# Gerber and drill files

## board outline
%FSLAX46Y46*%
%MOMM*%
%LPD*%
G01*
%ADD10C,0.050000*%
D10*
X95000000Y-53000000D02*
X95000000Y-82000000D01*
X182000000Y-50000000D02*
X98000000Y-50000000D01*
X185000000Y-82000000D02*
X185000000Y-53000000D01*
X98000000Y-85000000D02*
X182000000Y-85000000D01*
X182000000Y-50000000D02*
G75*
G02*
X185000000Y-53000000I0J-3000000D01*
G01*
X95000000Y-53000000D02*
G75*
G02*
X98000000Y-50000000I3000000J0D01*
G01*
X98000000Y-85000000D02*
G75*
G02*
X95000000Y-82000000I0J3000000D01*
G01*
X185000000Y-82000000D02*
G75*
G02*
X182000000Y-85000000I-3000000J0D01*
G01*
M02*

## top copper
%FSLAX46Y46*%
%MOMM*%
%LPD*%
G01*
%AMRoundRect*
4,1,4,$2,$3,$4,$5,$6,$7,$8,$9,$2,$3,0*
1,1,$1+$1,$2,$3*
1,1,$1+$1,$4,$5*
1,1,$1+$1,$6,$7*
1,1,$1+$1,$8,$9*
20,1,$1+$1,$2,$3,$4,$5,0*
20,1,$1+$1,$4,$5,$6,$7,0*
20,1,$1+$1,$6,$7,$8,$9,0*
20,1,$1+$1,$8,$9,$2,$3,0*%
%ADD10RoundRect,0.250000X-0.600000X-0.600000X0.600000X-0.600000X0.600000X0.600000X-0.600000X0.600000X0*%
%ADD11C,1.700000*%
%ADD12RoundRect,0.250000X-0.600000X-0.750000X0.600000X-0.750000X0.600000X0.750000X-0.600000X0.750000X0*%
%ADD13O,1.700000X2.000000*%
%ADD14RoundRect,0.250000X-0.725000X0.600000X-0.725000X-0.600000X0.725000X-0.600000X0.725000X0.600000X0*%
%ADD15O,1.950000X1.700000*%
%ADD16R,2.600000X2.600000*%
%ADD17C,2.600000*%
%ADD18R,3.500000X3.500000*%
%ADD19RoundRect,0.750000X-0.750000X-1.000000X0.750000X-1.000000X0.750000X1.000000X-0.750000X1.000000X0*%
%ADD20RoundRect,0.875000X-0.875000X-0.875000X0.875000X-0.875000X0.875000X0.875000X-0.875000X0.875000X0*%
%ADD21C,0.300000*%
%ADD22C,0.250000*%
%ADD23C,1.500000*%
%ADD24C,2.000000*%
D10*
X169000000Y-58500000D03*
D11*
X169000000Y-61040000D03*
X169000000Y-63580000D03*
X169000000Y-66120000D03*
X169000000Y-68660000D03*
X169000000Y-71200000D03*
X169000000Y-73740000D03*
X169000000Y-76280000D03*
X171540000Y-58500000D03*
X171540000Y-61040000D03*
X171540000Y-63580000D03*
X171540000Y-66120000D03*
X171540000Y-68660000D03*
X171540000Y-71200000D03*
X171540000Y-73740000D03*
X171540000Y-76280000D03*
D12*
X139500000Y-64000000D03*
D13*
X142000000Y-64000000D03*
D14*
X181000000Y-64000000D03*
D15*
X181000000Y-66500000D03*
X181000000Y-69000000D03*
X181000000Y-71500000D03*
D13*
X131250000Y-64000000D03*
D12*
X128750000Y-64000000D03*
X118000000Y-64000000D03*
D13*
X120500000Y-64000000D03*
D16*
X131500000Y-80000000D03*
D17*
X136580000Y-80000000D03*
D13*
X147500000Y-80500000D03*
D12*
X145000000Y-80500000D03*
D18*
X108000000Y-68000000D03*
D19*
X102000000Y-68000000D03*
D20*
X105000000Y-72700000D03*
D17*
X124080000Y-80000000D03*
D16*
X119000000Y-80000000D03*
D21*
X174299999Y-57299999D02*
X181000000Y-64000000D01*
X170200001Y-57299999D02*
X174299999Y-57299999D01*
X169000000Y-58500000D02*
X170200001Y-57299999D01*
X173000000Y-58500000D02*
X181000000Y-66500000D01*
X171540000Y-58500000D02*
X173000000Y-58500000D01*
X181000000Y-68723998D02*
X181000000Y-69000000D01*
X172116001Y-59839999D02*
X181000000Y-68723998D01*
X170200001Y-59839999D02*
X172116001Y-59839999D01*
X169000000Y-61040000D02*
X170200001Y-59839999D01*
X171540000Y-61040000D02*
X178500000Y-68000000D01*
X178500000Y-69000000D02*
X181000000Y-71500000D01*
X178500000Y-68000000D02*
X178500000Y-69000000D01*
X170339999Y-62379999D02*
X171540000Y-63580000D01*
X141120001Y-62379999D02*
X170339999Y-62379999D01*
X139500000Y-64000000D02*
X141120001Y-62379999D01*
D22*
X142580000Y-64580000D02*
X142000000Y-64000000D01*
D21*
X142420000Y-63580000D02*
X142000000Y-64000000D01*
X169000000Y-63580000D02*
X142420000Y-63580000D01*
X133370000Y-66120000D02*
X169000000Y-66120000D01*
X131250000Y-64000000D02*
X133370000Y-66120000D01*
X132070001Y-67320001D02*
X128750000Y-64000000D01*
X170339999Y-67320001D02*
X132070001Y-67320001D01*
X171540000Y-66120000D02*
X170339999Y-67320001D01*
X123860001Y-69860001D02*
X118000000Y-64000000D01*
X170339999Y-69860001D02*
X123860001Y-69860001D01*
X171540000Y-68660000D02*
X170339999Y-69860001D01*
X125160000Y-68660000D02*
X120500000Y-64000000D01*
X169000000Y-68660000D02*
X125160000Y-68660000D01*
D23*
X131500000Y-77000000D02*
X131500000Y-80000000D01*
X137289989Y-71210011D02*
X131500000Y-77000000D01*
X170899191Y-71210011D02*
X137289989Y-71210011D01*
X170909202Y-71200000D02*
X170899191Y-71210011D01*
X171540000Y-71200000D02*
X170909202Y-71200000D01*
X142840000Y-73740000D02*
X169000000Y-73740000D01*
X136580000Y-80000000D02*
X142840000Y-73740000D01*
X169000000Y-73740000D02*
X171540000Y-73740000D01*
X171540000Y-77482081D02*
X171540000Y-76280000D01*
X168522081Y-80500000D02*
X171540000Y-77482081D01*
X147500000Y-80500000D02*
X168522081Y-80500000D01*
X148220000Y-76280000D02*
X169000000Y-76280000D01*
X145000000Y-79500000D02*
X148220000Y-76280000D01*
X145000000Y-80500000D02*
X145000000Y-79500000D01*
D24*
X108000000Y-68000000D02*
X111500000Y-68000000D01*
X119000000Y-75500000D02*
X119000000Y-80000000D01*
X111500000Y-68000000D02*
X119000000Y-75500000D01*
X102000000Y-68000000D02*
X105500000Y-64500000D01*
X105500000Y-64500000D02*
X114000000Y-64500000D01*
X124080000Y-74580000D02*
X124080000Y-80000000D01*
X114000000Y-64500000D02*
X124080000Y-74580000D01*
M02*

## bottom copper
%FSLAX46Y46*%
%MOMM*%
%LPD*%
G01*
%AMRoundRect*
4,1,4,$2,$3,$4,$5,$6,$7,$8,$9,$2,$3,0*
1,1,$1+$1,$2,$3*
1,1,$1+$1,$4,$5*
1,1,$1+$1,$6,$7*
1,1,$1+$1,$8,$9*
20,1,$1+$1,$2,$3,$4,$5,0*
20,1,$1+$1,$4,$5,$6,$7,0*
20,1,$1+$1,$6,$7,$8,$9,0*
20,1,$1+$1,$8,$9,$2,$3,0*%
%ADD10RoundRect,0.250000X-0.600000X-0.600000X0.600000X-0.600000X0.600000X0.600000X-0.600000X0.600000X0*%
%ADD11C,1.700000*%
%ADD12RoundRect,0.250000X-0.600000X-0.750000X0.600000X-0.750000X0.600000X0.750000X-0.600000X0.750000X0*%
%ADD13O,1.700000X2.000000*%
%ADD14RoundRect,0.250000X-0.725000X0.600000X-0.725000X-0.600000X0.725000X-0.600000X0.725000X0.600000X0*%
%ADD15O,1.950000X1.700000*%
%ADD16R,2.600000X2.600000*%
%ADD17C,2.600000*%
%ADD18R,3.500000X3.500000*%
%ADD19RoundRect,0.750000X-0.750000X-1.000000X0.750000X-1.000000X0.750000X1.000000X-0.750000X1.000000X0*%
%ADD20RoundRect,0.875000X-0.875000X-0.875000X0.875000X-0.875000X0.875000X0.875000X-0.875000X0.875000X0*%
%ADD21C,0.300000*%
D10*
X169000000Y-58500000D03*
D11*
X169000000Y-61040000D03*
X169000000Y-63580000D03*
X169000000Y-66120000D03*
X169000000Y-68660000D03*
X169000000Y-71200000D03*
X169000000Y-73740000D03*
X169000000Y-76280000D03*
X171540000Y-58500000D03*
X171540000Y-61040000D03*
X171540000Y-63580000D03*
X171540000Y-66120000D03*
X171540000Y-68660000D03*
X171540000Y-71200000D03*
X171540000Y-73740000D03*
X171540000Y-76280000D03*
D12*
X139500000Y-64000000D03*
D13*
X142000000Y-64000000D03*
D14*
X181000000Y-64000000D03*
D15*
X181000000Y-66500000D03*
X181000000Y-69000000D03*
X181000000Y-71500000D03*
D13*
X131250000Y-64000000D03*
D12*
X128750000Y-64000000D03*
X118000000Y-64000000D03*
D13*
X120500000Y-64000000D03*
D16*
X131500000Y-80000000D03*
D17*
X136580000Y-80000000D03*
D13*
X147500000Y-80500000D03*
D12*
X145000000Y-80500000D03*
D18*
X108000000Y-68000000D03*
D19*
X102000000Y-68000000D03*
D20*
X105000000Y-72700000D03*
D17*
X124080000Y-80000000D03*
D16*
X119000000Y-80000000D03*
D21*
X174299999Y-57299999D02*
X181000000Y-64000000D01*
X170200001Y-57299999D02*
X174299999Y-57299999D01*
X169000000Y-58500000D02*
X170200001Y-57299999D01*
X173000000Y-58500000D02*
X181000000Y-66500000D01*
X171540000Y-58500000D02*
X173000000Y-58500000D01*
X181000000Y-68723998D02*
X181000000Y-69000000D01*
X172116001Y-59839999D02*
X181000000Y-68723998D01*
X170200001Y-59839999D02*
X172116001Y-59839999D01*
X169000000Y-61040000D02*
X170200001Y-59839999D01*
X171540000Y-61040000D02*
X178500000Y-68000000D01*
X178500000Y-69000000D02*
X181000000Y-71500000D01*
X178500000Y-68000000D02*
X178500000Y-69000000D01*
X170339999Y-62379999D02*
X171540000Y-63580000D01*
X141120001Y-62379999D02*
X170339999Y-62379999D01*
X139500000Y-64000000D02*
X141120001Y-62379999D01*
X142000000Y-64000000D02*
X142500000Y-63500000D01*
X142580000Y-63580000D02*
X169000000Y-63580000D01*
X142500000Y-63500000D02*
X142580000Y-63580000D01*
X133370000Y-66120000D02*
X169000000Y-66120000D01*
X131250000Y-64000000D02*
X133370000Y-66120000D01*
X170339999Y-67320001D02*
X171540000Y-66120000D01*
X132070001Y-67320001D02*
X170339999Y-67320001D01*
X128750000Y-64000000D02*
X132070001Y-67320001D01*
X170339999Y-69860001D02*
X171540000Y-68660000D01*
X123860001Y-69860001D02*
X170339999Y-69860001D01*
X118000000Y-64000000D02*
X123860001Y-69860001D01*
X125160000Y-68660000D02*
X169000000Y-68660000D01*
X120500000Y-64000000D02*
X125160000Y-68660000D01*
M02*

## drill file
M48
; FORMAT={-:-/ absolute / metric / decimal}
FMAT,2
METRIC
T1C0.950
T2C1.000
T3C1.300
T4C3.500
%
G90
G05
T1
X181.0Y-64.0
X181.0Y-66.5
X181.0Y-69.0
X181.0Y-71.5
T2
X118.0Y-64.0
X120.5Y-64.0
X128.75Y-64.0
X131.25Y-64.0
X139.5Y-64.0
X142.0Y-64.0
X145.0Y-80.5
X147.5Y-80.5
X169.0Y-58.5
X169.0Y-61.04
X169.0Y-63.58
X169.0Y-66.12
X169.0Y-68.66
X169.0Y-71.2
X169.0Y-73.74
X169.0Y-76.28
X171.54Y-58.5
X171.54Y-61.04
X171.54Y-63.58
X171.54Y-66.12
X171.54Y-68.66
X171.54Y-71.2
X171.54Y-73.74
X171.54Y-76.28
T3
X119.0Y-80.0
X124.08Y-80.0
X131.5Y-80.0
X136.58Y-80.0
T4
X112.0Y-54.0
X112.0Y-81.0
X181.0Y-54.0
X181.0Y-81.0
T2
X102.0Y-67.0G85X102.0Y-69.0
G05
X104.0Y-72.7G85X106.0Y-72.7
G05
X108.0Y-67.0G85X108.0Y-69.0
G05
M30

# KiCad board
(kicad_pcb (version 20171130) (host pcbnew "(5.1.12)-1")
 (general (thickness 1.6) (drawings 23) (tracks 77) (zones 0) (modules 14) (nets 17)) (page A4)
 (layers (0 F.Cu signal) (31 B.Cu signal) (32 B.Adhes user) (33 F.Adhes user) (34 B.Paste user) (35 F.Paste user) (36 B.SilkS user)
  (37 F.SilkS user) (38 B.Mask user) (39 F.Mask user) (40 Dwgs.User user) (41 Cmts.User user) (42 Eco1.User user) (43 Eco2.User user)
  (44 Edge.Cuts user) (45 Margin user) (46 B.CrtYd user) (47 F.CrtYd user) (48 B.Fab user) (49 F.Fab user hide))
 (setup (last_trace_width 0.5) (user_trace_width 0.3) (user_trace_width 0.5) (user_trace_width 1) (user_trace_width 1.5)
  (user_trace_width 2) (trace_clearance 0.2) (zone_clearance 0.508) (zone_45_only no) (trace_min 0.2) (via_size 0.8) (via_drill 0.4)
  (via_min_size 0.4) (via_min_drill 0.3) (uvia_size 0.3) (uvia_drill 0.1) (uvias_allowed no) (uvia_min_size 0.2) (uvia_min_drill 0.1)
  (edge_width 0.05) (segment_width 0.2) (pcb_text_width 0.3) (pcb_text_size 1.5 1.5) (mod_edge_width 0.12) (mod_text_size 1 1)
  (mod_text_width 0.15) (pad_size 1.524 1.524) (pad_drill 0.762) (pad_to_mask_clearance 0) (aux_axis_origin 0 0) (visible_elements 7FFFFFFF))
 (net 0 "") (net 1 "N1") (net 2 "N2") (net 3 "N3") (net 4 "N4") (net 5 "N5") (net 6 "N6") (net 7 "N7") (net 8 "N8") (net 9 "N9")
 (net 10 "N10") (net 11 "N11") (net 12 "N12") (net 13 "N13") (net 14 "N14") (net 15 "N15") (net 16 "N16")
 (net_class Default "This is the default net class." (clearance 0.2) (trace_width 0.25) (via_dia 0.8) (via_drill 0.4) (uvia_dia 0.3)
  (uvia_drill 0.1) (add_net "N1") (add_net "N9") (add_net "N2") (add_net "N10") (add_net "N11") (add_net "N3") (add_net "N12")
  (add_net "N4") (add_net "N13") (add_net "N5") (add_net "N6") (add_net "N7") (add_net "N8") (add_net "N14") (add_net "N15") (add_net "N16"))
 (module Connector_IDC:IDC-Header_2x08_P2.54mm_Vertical (layer F.Cu) (at 169 58.5)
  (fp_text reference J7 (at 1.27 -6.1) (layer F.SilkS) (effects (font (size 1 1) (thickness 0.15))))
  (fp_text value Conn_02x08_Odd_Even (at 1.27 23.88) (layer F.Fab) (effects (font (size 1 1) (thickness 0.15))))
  (pad 1 thru_hole roundrect (at 0 0) (size 1.7 1.7) (drill 1) (layers *.Cu *.Mask) (roundrect_rratio 0.1470588235294118) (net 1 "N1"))
  (pad 3 thru_hole circle (at 0 2.54) (size 1.7 1.7) (drill 1) (layers *.Cu *.Mask) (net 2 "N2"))
  (pad 5 thru_hole circle (at 0 5.08) (size 1.7 1.7) (drill 1) (layers *.Cu *.Mask) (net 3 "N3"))
  (pad 7 thru_hole circle (at 0 7.62) (size 1.7 1.7) (drill 1) (layers *.Cu *.Mask) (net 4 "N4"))
  (pad 9 thru_hole circle (at 0 10.16) (size 1.7 1.7) (drill 1) (layers *.Cu *.Mask) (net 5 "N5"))
  (pad 11 thru_hole circle (at 0 12.7) (size 1.7 1.7) (drill 1) (layers *.Cu *.Mask) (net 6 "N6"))
  (pad 13 thru_hole circle (at 0 15.24) (size 1.7 1.7) (drill 1) (layers *.Cu *.Mask) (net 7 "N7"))
  (pad 15 thru_hole circle (at 0 17.78) (size 1.7 1.7) (drill 1) (layers *.Cu *.Mask) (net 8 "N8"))
  (pad 2 thru_hole circle (at 2.54 0) (size 1.7 1.7) (drill 1) (layers *.Cu *.Mask) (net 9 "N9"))
  (pad 4 thru_hole circle (at 2.54 2.54) (size 1.7 1.7) (drill 1) (layers *.Cu *.Mask) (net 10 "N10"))
  (pad 6 thru_hole circle (at 2.54 5.08) (size 1.7 1.7) (drill 1) (layers *.Cu *.Mask) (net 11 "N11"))
  (pad 8 thru_hole circle (at 2.54 7.62) (size 1.7 1.7) (drill 1) (layers *.Cu *.Mask) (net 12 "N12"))
  (pad 10 thru_hole circle (at 2.54 10.16) (size 1.7 1.7) (drill 1) (layers *.Cu *.Mask) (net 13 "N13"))
  (pad 12 thru_hole circle (at 2.54 12.7) (size 1.7 1.7) (drill 1) (layers *.Cu *.Mask) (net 6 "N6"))
  (pad 14 thru_hole circle (at 2.54 15.24) (size 1.7 1.7) (drill 1) (layers *.Cu *.Mask) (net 7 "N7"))
  (pad 16 thru_hole circle (at 2.54 17.78) (size 1.7 1.7) (drill 1) (layers *.Cu *.Mask) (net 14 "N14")))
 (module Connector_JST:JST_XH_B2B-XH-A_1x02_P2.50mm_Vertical (layer F.Cu) (at 139.5 64)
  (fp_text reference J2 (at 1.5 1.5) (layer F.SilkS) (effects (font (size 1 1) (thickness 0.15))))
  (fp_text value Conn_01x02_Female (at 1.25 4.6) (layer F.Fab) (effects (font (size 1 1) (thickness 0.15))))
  (pad 1 thru_hole roundrect (at 0 0) (size 1.7 2) (drill 1) (layers *.Cu *.Mask) (roundrect_rratio 0.1470588235294118) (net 11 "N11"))
  (pad 2 thru_hole oval (at 2.5 0) (size 1.7 2) (drill 1) (layers *.Cu *.Mask) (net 3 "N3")))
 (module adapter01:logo (layer F.Cu) (at 155.5 67.5)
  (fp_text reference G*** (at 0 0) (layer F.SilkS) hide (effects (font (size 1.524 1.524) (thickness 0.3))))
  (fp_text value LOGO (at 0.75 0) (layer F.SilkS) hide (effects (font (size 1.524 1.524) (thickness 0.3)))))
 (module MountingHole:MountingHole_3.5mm (layer F.Cu) (at 181 54)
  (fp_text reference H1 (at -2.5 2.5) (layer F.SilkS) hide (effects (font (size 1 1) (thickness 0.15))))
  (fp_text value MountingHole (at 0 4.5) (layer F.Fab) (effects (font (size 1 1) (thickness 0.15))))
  (pad 1 np_thru_hole circle (at 0 0) (size 3.5 3.5) (drill 3.5) (layers *.Cu *.Mask)))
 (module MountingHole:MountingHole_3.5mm (layer F.Cu) (at 112 81)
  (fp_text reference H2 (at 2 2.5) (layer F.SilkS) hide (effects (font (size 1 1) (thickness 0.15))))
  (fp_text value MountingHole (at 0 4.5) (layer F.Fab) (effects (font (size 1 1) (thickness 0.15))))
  (pad 1 np_thru_hole circle (at 0 0) (size 3.5 3.5) (drill 3.5) (layers *.Cu *.Mask)))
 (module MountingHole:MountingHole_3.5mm (layer F.Cu) (at 181 81)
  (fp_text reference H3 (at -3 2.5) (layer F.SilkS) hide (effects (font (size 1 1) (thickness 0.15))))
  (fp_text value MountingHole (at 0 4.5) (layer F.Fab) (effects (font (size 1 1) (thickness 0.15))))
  (pad 1 np_thru_hole circle (at 0 0) (size 3.5 3.5) (drill 3.5) (layers *.Cu *.Mask)))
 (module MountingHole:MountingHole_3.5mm (layer F.Cu) (at 112 54)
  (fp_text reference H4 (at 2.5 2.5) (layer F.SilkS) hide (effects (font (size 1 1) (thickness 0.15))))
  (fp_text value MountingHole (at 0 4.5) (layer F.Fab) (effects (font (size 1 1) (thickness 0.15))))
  (pad 1 np_thru_hole circle (at 0 0) (size 3.5 3.5) (drill 3.5) (layers *.Cu *.Mask)))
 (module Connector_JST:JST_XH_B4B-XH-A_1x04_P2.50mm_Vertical (layer F.Cu) (at 181 64 270)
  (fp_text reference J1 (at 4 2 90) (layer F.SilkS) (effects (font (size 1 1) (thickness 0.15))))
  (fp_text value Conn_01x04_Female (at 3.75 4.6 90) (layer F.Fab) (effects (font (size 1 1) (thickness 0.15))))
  (pad 1 thru_hole roundrect (at 0 0 270) (size 1.7 1.95) (drill 0.95) (layers *.Cu *.Mask) (roundrect_rratio 0.1470588235294118)
   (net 1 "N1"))
  (pad 2 thru_hole oval (at 2.5 0 270) (size 1.7 1.95) (drill 0.95) (layers *.Cu *.Mask) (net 9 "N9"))
  (pad 3 thru_hole oval (at 5 0 270) (size 1.7 1.95) (drill 0.95) (layers *.Cu *.Mask) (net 2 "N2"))
  (pad 4 thru_hole oval (at 7.5 0 270) (size 1.7 1.95) (drill 0.95) (layers *.Cu *.Mask) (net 10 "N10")))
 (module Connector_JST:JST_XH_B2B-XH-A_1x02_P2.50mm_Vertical (layer F.Cu) (at 128.75 64)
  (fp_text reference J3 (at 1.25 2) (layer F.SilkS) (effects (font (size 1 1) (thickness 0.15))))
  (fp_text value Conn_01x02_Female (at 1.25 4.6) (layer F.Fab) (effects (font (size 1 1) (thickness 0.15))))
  (pad 2 thru_hole oval (at 2.5 0) (size 1.7 2) (drill 1) (layers *.Cu *.Mask) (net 4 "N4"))
  (pad 1 thru_hole roundrect (at 0 0) (size 1.7 2) (drill 1) (layers *.Cu *.Mask) (roundrect_rratio 0.1470588235294118) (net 12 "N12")))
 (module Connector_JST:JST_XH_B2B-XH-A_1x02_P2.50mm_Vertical (layer F.Cu) (at 118 64)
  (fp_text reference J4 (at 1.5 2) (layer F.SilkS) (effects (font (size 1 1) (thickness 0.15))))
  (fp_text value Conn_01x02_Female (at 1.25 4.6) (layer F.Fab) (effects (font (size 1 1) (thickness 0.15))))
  (pad 1 thru_hole roundrect (at 0 0) (size 1.7 2) (drill 1) (layers *.Cu *.Mask) (roundrect_rratio 0.1470588235294118) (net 13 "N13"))
  (pad 2 thru_hole oval (at 2.5 0) (size 1.7 2) (drill 1) (layers *.Cu *.Mask) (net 5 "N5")))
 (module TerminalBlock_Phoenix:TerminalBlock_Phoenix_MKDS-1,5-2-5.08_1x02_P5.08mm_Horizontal (layer F.Cu) (at 131.5 80)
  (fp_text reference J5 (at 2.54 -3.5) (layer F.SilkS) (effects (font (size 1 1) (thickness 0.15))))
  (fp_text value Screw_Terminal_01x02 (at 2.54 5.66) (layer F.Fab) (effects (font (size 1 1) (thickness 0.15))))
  (pad 1 thru_hole rect (at 0 0) (size 2.6 2.6) (drill 1.3) (layers *.Cu *.Mask) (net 6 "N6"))
  (pad 2 thru_hole circle (at 5.08 0) (size 2.6 2.6) (drill 1.3) (layers *.Cu *.Mask) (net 7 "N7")))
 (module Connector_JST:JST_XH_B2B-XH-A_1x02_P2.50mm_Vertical (layer F.Cu) (at 145 80.5)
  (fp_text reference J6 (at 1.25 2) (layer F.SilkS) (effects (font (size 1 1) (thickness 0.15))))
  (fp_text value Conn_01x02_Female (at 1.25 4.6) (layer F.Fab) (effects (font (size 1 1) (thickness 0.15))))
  (pad 2 thru_hole oval (at 2.5 0) (size 1.7 2) (drill 1) (layers *.Cu *.Mask) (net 14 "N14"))
  (pad 1 thru_hole roundrect (at 0 0) (size 1.7 2) (drill 1) (layers *.Cu *.Mask) (roundrect_rratio 0.1470588235294118) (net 8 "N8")))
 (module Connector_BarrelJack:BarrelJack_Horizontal (layer F.Cu) (at 108 68)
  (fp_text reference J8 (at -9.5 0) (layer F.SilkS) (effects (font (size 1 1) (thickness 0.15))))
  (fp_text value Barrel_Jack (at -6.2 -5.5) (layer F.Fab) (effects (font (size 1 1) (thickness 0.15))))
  (pad 1 thru_hole rect (at 0 0) (size 3.5 3.5) (drill oval 1 3) (layers *.Cu *.Mask) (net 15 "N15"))
  (pad 2 thru_hole roundrect (at -6 0) (size 3 3.5) (drill oval 1 3) (layers *.Cu *.Mask) (roundrect_rratio 0.25) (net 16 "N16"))
  (pad 3 thru_hole roundrect (at -3 4.7) (size 3.5 3.5) (drill oval 3 1) (layers *.Cu *.Mask) (roundrect_rratio 0.25)))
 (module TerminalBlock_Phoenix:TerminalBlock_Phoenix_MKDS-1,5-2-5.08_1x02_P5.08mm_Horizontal (layer F.Cu) (at 119 80)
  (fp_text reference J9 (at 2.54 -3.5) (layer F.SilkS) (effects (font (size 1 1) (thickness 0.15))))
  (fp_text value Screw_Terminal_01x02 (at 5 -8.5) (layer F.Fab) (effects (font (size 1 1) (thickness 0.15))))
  (pad 2 thru_hole circle (at 5.08 0) (size 2.6 2.6) (drill 1.3) (layers *.Cu *.Mask) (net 16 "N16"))
  (pad 1 thru_hole rect (at 0 0) (size 2.6 2.6) (drill 1.3) (layers *.Cu *.Mask) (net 15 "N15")))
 (gr_line (start 95 53) (end 95 82) (layer Edge.Cuts) (width 0.05))
 (gr_line (start 182 50) (end 98 50) (layer Edge.Cuts) (width 0.05))
 (gr_line (start 185 82) (end 185 53) (layer Edge.Cuts) (width 0.05))
 (gr_line (start 98 85) (end 182 85) (layer Edge.Cuts) (width 0.05))
 (gr_arc (start 182 53) (end 185 53) (angle -90) (layer Edge.Cuts) (width 0.05))
 (gr_arc (start 98 53) (end 98 50) (angle -90) (layer Edge.Cuts) (width 0.05))
 (gr_arc (start 98 82) (end 95 82) (angle -90) (layer Edge.Cuts) (width 0.05))
 (gr_arc (start 182 82) (end 182 85) (angle -90) (layer Edge.Cuts) (width 0.05))
 (segment (start 174.299999 57.299999) (end 181 64) (width 0.3) (layer F.Cu) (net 1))
 (segment (start 170.200001 57.299999) (end 174.299999 57.299999) (width 0.3) (layer F.Cu) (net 1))
 (segment (start 169 58.5) (end 170.200001 57.299999) (width 0.3) (layer F.Cu) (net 1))
 (segment (start 174.299999 57.299999) (end 181 64) (width 0.3) (layer B.Cu) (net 1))
 (segment (start 170.200001 57.299999) (end 174.299999 57.299999) (width 0.3) (layer B.Cu) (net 1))
 (segment (start 169 58.5) (end 170.200001 57.299999) (width 0.3) (layer B.Cu) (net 1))
 (segment (start 173 58.5) (end 181 66.5) (width 0.3) (layer F.Cu) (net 9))
 (segment (start 171.54 58.5) (end 173 58.5) (width 0.3) (layer F.Cu) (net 9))
 (segment (start 173 58.5) (end 181 66.5) (width 0.3) (layer B.Cu) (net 9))
 (segment (start 171.54 58.5) (end 173 58.5) (width 0.3) (layer B.Cu) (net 9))
 (segment (start 181 68.723998) (end 181 69) (width 0.3) (layer B.Cu) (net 2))
 (segment (start 172.116001 59.839999) (end 181 68.723998) (width 0.3) (layer B.Cu) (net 2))
 (segment (start 170.200001 59.839999) (end 172.116001 59.839999) (width 0.3) (layer B.Cu) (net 2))
 (segment (start 169 61.04) (end 170.200001 59.839999) (width 0.3) (layer B.Cu) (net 2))
 (segment (start 181 68.723998) (end 181 69) (width 0.3) (layer F.Cu) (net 2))
 (segment (start 172.116001 59.839999) (end 181 68.723998) (width 0.3) (layer F.Cu) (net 2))
 (segment (start 170.200001 59.839999) (end 172.116001 59.839999) (width 0.3) (layer F.Cu) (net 2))
 (segment (start 169 61.04) (end 170.200001 59.839999) (width 0.3) (layer F.Cu) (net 2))
 (segment (start 171.54 61.04) (end 178.5 68) (width 0.3) (layer F.Cu) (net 10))
 (segment (start 178.5 69) (end 181 71.5) (width 0.3) (layer F.Cu) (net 10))
 (segment (start 178.5 68) (end 178.5 69) (width 0.3) (layer F.Cu) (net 10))
 (segment (start 171.54 61.04) (end 178.5 68) (width 0.3) (layer B.Cu) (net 10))
 (segment (start 178.5 69) (end 181 71.5) (width 0.3) (layer B.Cu) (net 10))
 (segment (start 178.5 68) (end 178.5 69) (width 0.3) (layer B.Cu) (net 10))
 (segment (start 170.339999 62.379999) (end 171.54 63.58) (width 0.3) (layer F.Cu) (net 11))
 (segment (start 141.120001 62.379999) (end 170.339999 62.379999) (width 0.3) (layer F.Cu) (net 11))
 (segment (start 139.5 64) (end 141.120001 62.379999) (width 0.3) (layer F.Cu) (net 11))
 (segment (start 170.339999 62.379999) (end 171.54 63.58) (width 0.3) (layer B.Cu) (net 11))
 (segment (start 141.120001 62.379999) (end 170.339999 62.379999) (width 0.3) (layer B.Cu) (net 11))
 (segment (start 139.5 64) (end 141.120001 62.379999) (width 0.3) (layer B.Cu) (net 11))
 (segment (start 142.58 64.58) (end 142 64) (width 0.25) (layer F.Cu) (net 3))
 (segment (start 142.42 63.58) (end 142 64) (width 0.3) (layer F.Cu) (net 3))
 (segment (start 169 63.58) (end 142.42 63.58) (width 0.3) (layer F.Cu) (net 3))
 (segment (start 142 64) (end 142.5 63.5) (width 0.3) (layer B.Cu) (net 3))
 (segment (start 142.58 63.58) (end 169 63.58) (width 0.3) (layer B.Cu) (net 3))
 (segment (start 142.5 63.5) (end 142.58 63.58) (width 0.3) (layer B.Cu) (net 3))
 (segment (start 133.37 66.12) (end 169 66.12) (width 0.3) (layer B.Cu) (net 4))
 (segment (start 131.25 64) (end 133.37 66.12) (width 0.3) (layer B.Cu) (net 4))
 (segment (start 133.37 66.12) (end 169 66.12) (width 0.3) (layer F.Cu) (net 4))
 (segment (start 131.25 64) (end 133.37 66.12) (width 0.3) (layer F.Cu) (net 4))
 (segment (start 132.070001 67.320001) (end 128.75 64) (width 0.3) (layer F.Cu) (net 12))
 (segment (start 170.339999 67.320001) (end 132.070001 67.320001) (width 0.3) (layer F.Cu) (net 12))
 (segment (start 171.54 66.12) (end 170.339999 67.320001) (width 0.3) (layer F.Cu) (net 12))
 (segment (start 170.339999 67.320001) (end 171.54 66.12) (width 0.3) (layer B.Cu) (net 12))
 (segment (start 132.070001 67.320001) (end 170.339999 67.320001) (width 0.3) (layer B.Cu) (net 12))
 (segment (start 128.75 64) (end 132.070001 67.320001) (width 0.3) (layer B.Cu) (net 12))
 (segment (start 123.860001 69.860001) (end 118 64) (width 0.3) (layer F.Cu) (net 13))
 (segment (start 170.339999 69.860001) (end 123.860001 69.860001) (width 0.3) (layer F.Cu) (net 13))
 (segment (start 171.54 68.66) (end 170.339999 69.860001) (width 0.3) (layer F.Cu) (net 13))
 (segment (start 170.339999 69.860001) (end 171.54 68.66) (width 0.3) (layer B.Cu) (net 13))
 (segment (start 123.860001 69.860001) (end 170.339999 69.860001) (width 0.3) (layer B.Cu) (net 13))
 (segment (start 118 64) (end 123.860001 69.860001) (width 0.3) (layer B.Cu) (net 13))
 (segment (start 125.16 68.66) (end 120.5 64) (width 0.3) (layer F.Cu) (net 5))
 (segment (start 169 68.66) (end 125.16 68.66) (width 0.3) (layer F.Cu) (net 5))
 (segment (start 125.16 68.66) (end 169 68.66) (width 0.3) (layer B.Cu) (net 5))
 (segment (start 120.5 64) (end 125.16 68.66) (width 0.3) (layer B.Cu) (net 5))
 (segment (start 131.5 77) (end 131.5 80) (width 1.5) (layer F.Cu) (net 6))
 (segment (start 137.289989 71.210011) (end 131.5 77) (width 1.5) (layer F.Cu) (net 6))
 (segment (start 170.899191 71.210011) (end 137.289989 71.210011) (width 1.5) (layer F.Cu) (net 6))
 (segment (start 170.909202 71.2) (end 170.899191 71.210011) (width 1.5) (layer F.Cu) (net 6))
 (segment (start 171.54 71.2) (end 170.909202 71.2) (width 1.5) (layer F.Cu) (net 6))
 (segment (start 142.84 73.74) (end 169 73.74) (width 1.5) (layer F.Cu) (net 7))
 (segment (start 136.58 80) (end 142.84 73.74) (width 1.5) (layer F.Cu) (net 7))
 (segment (start 169 73.74) (end 171.54 73.74) (width 1.5) (layer F.Cu) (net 7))
 (segment (start 171.54 77.482081) (end 171.54 76.28) (width 1.5) (layer F.Cu) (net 14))
 (segment (start 168.522081 80.5) (end 171.54 77.482081) (width 1.5) (layer F.Cu) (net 14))
 (segment (start 147.5 80.5) (end 168.522081 80.5) (width 1.5) (layer F.Cu) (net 14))
 (segment (start 148.22 76.28) (end 169 76.28) (width 1.5) (layer F.Cu) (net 8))
 (segment (start 145 79.5) (end 148.22 76.28) (width 1.5) (layer F.Cu) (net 8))
 (segment (start 145 80.5) (end 145 79.5) (width 1.5) (layer F.Cu) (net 8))
 (segment (start 108 68) (end 111.5 68) (width 2) (layer F.Cu) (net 15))
 (segment (start 119 75.5) (end 119 80) (width 2) (layer F.Cu) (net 15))
 (segment (start 111.5 68) (end 119 75.5) (width 2) (layer F.Cu) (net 15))
 (segment (start 102 68) (end 105.5 64.5) (width 2) (layer F.Cu) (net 16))
 (segment (start 105.5 64.5) (end 114 64.5) (width 2) (layer F.Cu) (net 16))
 (segment (start 124.08 74.58) (end 124.08 80) (width 2) (layer F.Cu) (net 16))
 (segment (start 114 64.5) (end 124.08 74.58) (width 2) (layer F.Cu) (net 16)))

